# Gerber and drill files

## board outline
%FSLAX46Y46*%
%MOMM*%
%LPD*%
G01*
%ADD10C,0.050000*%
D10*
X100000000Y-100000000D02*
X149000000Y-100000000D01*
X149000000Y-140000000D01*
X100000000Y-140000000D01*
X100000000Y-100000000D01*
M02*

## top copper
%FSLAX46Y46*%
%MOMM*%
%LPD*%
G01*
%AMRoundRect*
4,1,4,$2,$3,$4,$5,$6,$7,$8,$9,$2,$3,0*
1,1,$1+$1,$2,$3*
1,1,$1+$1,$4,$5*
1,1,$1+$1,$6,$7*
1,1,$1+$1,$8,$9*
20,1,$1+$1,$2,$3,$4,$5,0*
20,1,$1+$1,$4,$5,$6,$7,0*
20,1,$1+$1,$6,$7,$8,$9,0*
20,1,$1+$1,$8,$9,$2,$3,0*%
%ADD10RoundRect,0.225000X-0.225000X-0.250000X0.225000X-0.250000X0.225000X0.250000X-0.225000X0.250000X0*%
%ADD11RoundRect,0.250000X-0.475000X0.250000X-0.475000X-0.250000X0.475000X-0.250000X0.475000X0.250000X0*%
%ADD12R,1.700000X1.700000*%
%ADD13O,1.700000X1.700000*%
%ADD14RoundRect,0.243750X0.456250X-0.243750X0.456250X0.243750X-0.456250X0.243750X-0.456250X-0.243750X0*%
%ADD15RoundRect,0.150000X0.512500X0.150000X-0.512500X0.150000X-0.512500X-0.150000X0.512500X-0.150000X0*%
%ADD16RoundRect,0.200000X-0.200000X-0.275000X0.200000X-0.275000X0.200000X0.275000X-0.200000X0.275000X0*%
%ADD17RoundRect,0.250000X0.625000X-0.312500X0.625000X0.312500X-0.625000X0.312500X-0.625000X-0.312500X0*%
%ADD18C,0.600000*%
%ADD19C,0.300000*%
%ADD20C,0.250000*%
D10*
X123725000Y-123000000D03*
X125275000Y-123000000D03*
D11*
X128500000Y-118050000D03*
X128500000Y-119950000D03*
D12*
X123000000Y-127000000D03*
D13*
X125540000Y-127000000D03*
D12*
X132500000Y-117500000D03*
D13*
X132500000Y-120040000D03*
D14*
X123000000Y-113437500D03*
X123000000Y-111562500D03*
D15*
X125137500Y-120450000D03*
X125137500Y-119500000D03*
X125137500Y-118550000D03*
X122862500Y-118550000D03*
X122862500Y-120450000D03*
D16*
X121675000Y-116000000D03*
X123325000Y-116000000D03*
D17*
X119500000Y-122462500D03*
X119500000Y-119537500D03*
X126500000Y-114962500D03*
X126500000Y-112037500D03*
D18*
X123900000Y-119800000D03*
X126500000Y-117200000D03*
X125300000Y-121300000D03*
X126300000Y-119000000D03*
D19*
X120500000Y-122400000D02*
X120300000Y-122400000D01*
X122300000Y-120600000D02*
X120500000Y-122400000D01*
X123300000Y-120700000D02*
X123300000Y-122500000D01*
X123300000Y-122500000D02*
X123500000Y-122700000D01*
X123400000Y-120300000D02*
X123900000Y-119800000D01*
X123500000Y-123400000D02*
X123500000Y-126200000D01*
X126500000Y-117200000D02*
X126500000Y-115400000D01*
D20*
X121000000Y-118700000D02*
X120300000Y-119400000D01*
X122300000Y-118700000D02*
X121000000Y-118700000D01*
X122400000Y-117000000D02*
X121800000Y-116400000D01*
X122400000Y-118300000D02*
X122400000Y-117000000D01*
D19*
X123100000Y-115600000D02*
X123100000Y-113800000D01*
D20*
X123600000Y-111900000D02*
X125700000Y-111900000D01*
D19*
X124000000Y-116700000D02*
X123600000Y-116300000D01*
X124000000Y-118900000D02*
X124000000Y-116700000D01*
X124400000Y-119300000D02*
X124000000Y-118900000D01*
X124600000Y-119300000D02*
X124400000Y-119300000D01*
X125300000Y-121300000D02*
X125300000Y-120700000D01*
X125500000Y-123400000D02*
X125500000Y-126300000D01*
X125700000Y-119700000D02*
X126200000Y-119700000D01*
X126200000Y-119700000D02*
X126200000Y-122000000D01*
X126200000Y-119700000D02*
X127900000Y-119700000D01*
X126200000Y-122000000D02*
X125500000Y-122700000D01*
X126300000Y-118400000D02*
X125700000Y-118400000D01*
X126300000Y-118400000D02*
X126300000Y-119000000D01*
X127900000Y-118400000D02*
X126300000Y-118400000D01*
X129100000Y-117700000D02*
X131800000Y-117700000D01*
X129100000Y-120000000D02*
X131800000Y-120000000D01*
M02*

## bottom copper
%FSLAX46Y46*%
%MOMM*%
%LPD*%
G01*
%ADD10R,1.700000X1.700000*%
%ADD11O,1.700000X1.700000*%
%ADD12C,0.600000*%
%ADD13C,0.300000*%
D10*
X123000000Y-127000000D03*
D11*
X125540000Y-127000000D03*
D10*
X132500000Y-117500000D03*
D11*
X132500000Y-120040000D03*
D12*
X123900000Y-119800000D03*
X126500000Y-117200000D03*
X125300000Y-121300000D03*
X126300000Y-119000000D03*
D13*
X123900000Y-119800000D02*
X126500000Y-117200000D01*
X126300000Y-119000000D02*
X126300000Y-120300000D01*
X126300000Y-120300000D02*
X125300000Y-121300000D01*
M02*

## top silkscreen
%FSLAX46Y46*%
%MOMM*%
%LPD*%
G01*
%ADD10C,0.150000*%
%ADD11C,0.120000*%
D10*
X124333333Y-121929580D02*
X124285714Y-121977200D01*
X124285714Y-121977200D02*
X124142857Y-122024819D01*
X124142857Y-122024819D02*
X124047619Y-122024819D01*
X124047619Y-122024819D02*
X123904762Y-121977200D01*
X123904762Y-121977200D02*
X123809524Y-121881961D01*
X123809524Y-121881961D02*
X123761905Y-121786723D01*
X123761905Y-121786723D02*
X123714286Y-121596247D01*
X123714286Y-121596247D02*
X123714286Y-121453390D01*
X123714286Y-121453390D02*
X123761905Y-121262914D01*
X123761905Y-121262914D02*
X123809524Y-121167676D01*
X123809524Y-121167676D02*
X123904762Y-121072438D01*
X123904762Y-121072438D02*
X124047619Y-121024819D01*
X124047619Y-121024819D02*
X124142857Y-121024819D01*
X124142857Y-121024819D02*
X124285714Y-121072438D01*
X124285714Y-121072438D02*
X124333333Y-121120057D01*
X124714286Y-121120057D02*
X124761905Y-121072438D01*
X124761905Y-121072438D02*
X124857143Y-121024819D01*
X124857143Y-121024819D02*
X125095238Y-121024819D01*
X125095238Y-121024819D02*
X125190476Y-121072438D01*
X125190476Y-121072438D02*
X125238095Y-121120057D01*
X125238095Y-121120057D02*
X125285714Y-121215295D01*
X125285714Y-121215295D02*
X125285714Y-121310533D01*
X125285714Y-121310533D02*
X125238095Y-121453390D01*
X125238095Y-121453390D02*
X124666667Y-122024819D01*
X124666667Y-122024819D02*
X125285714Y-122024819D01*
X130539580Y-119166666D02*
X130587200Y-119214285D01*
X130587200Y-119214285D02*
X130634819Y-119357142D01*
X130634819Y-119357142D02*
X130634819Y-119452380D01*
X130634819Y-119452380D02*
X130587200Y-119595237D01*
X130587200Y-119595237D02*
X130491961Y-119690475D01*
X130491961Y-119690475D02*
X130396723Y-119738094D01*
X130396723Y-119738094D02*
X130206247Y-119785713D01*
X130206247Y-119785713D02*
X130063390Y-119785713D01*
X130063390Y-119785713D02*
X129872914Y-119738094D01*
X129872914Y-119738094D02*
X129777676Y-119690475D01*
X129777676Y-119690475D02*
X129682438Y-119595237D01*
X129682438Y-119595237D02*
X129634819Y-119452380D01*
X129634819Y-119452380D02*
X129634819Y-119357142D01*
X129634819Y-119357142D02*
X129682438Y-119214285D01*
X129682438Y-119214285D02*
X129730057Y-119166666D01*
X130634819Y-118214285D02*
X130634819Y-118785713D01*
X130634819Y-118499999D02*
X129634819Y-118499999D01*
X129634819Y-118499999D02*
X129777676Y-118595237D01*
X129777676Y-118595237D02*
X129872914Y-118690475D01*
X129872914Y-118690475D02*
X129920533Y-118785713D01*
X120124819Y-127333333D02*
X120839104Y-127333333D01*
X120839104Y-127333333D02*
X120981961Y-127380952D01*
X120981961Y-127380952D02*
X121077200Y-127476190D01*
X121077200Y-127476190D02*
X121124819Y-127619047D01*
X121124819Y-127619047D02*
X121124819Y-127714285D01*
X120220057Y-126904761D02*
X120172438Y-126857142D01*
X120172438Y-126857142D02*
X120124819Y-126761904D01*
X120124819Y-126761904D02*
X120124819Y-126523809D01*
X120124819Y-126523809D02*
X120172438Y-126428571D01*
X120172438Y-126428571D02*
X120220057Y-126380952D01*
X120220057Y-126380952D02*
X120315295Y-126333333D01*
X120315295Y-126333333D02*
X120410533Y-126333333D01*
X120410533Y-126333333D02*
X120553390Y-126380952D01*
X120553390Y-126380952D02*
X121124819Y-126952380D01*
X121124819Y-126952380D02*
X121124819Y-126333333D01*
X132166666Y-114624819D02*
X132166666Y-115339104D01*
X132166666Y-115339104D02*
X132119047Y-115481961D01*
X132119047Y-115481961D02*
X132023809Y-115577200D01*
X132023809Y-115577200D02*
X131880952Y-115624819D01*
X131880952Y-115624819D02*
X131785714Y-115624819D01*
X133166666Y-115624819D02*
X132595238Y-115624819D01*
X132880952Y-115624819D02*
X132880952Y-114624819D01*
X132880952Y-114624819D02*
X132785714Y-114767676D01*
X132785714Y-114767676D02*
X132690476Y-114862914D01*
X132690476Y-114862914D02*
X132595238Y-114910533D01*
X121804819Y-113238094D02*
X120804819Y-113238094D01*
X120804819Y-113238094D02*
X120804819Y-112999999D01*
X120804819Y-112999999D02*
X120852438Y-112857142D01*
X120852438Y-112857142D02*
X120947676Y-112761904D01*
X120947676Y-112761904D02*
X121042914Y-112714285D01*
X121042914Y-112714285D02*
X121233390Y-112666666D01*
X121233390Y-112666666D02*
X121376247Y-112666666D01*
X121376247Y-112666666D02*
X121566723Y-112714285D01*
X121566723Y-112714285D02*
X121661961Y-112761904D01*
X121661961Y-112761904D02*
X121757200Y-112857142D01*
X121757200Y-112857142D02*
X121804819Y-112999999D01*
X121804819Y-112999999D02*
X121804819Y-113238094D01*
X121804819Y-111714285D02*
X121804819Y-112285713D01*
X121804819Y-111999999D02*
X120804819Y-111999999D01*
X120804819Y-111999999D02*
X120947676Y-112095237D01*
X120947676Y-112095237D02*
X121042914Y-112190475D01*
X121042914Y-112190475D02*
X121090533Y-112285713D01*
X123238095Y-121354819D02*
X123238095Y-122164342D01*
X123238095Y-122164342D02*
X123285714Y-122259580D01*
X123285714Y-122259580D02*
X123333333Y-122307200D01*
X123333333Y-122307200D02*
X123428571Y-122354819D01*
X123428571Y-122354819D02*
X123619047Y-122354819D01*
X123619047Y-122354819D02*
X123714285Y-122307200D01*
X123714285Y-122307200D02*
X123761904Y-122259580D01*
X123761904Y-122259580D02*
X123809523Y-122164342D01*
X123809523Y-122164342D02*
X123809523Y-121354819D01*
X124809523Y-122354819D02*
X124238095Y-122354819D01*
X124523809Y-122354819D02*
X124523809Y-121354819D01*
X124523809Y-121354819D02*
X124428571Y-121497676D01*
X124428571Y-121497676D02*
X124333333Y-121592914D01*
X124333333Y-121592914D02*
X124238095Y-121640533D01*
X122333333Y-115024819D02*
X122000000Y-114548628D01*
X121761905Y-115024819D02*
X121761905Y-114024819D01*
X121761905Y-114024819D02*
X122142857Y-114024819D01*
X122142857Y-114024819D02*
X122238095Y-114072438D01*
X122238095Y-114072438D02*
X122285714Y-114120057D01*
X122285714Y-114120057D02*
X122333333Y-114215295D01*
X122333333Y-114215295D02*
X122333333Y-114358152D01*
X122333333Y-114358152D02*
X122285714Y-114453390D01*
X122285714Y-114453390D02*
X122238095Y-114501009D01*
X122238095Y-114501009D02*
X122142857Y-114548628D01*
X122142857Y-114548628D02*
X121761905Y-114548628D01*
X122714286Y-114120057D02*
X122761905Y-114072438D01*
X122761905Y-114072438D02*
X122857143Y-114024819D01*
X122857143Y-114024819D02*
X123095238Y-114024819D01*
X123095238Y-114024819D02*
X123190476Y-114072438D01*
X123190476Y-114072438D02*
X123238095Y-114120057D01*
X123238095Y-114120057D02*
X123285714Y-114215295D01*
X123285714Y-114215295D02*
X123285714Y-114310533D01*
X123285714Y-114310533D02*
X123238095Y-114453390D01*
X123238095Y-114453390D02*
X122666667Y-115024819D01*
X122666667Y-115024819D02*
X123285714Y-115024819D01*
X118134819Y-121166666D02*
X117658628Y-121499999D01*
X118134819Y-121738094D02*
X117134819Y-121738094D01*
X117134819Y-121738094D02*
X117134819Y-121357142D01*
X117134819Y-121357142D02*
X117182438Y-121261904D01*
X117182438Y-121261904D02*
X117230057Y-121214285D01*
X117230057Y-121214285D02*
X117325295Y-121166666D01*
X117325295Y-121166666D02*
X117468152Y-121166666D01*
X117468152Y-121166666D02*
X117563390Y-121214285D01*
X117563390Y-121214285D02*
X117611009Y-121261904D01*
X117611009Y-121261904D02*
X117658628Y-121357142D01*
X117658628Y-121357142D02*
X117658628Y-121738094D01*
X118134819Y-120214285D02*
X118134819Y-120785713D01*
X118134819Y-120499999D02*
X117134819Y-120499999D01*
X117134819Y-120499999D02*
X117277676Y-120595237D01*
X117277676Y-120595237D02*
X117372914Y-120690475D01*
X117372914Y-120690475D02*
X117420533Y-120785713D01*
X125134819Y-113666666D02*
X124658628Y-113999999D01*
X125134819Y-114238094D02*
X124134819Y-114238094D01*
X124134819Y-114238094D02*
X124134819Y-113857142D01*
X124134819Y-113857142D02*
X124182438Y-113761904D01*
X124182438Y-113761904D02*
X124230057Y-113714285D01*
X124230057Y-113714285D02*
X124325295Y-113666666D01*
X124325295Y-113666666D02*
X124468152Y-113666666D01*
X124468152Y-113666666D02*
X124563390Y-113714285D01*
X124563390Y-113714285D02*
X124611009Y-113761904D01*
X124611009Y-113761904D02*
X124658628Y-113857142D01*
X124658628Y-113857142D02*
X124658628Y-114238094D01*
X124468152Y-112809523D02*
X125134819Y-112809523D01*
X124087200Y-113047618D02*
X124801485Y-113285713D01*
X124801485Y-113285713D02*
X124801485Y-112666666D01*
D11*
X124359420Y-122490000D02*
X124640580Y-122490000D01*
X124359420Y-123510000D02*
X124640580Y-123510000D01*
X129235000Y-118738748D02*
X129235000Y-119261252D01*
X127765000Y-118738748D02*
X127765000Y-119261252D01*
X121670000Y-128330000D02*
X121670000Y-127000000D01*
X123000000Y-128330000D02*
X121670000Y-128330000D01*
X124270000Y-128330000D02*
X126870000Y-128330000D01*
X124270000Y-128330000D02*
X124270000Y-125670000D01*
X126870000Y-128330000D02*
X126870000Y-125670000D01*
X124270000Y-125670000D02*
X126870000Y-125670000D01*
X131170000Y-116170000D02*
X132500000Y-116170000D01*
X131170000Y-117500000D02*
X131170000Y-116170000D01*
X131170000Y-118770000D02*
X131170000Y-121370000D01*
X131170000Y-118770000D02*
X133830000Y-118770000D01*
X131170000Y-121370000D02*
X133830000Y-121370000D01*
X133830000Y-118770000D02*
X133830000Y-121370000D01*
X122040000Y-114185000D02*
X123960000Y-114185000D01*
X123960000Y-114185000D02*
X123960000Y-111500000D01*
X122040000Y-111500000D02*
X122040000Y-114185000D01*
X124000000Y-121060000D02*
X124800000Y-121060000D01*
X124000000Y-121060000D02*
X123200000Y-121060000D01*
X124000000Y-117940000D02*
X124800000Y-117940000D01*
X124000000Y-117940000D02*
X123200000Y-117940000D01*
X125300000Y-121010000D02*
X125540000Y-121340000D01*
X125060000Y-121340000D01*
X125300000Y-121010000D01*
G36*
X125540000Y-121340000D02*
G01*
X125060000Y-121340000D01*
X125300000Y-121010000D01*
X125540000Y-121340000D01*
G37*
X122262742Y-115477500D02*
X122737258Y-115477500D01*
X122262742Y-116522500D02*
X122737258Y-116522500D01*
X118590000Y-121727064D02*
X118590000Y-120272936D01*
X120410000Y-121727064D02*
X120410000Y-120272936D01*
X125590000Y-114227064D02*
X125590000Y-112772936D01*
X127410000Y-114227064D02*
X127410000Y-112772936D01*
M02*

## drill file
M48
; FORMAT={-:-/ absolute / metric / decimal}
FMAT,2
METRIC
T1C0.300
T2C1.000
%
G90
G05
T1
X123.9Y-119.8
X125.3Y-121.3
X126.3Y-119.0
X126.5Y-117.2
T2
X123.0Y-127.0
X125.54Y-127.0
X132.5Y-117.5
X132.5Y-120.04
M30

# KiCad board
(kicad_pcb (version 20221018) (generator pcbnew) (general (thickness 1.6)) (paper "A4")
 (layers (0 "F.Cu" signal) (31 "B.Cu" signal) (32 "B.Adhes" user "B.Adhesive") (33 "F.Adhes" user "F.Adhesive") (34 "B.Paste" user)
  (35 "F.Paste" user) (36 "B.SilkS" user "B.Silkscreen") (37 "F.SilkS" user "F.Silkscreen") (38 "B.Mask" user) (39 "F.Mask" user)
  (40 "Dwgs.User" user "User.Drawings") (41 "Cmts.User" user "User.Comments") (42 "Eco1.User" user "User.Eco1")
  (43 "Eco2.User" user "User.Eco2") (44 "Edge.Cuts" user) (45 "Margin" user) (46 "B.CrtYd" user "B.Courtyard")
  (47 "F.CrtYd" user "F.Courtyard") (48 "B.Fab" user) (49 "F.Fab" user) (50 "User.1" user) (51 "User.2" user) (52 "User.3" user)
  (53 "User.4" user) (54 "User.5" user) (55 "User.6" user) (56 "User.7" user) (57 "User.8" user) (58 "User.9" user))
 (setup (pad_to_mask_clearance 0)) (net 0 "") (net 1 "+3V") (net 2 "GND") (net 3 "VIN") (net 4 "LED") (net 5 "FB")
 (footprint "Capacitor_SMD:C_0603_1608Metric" (layer "F.Cu") (at 124.5 123)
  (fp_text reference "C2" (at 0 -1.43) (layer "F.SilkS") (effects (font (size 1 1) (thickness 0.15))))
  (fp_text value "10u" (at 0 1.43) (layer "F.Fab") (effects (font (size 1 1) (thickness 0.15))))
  (fp_line (start -0.14058 -0.51) (end 0.14058 -0.51) (stroke (width 0.12) (type solid)) (layer "F.SilkS"))
  (fp_line (start -0.14058 0.51) (end 0.14058 0.51) (stroke (width 0.12) (type solid)) (layer "F.SilkS"))
  (pad "1" smd roundrect (at -0.775 0) (size 0.9 0.95) (layers "F.Cu" "F.Paste" "F.Mask") (roundrect_rratio 0.25) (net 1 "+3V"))
  (pad "2" smd roundrect (at 0.775 0) (size 0.9 0.95) (layers "F.Cu" "F.Paste" "F.Mask") (roundrect_rratio 0.25) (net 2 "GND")))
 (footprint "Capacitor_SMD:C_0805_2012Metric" (layer "F.Cu") (at 128.5 119 -90)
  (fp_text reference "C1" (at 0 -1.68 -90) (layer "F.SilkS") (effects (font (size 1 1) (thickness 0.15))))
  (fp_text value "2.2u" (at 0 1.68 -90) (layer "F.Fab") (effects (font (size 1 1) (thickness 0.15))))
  (fp_line (start -0.261252 -0.735) (end 0.261252 -0.735) (stroke (width 0.12) (type solid)) (layer "F.SilkS"))
  (fp_line (start -0.261252 0.735) (end 0.261252 0.735) (stroke (width 0.12) (type solid)) (layer "F.SilkS"))
  (pad "1" smd roundrect (at -0.95 0 270) (size 1 1.45) (layers "F.Cu" "F.Paste" "F.Mask") (roundrect_rratio 0.25) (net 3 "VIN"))
  (pad "2" smd roundrect (at 0.95 0 270) (size 1 1.45) (layers "F.Cu" "F.Paste" "F.Mask") (roundrect_rratio 0.25) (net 2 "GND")))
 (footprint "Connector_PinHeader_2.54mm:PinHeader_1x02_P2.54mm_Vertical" (layer "F.Cu") (at 123 127 90)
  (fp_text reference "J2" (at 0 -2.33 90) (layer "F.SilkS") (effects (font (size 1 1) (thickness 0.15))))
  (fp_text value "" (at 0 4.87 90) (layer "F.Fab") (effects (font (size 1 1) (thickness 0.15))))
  (fp_line (start -1.33 -1.33) (end 0 -1.33) (stroke (width 0.12) (type solid)) (layer "F.SilkS"))
  (fp_line (start -1.33 0) (end -1.33 -1.33) (stroke (width 0.12) (type solid)) (layer "F.SilkS"))
  (fp_line (start -1.33 1.27) (end -1.33 3.87) (stroke (width 0.12) (type solid)) (layer "F.SilkS"))
  (fp_line (start -1.33 1.27) (end 1.33 1.27) (stroke (width 0.12) (type solid)) (layer "F.SilkS"))
  (fp_line (start -1.33 3.87) (end 1.33 3.87) (stroke (width 0.12) (type solid)) (layer "F.SilkS"))
  (fp_line (start 1.33 1.27) (end 1.33 3.87) (stroke (width 0.12) (type solid)) (layer "F.SilkS"))
  (pad "1" thru_hole rect (at 0 0 90) (size 1.7 1.7) (drill 1) (layers "*.Cu" "*.Mask") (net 1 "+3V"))
  (pad "2" thru_hole oval (at 0 2.54 90) (size 1.7 1.7) (drill 1) (layers "*.Cu" "*.Mask") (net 2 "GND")))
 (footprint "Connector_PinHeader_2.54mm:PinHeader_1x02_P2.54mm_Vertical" (layer "F.Cu") (at 132.5 117.5)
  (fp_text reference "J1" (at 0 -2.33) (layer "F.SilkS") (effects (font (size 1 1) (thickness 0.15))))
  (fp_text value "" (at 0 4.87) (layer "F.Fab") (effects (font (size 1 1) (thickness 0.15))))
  (fp_line (start -1.33 -1.33) (end 0 -1.33) (stroke (width 0.12) (type solid)) (layer "F.SilkS"))
  (fp_line (start -1.33 0) (end -1.33 -1.33) (stroke (width 0.12) (type solid)) (layer "F.SilkS"))
  (fp_line (start -1.33 1.27) (end -1.33 3.87) (stroke (width 0.12) (type solid)) (layer "F.SilkS"))
  (fp_line (start -1.33 1.27) (end 1.33 1.27) (stroke (width 0.12) (type solid)) (layer "F.SilkS"))
  (fp_line (start -1.33 3.87) (end 1.33 3.87) (stroke (width 0.12) (type solid)) (layer "F.SilkS"))
  (fp_line (start 1.33 1.27) (end 1.33 3.87) (stroke (width 0.12) (type solid)) (layer "F.SilkS"))
  (pad "1" thru_hole rect (at 0 0) (size 1.7 1.7) (drill 1) (layers "*.Cu" "*.Mask") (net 3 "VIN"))
  (pad "2" thru_hole oval (at 0 2.54) (size 1.7 1.7) (drill 1) (layers "*.Cu" "*.Mask") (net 2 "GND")))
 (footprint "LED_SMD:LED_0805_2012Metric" (layer "F.Cu") (at 123 112.5 90)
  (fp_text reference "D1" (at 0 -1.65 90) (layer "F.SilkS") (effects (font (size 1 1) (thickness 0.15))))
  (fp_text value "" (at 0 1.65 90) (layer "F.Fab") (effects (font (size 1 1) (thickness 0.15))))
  (fp_line (start -1.685 -0.96) (end -1.685 0.96) (stroke (width 0.12) (type solid)) (layer "F.SilkS"))
  (fp_line (start -1.685 0.96) (end 1 0.96) (stroke (width 0.12) (type solid)) (layer "F.SilkS"))
  (fp_line (start 1 -0.96) (end -1.685 -0.96) (stroke (width 0.12) (type solid)) (layer "F.SilkS"))
  (pad "1" smd roundrect (at -0.9375 0 90) (size 0.975 1.4) (layers "F.Cu" "F.Paste" "F.Mask") (roundrect_rratio 0.25) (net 2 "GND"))
  (pad "2" smd roundrect (at 0.9375 0 90) (size 0.975 1.4) (layers "F.Cu" "F.Paste" "F.Mask") (roundrect_rratio 0.25) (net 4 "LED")))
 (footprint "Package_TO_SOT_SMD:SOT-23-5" (layer "F.Cu") (at 124 119.5 180)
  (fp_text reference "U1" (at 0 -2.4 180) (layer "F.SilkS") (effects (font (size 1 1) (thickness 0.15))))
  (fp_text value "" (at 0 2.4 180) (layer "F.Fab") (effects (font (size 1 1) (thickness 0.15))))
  (fp_line (start 0 -1.56) (end -0.8 -1.56) (stroke (width 0.12) (type solid)) (layer "F.SilkS"))
  (fp_line (start 0 -1.56) (end 0.8 -1.56) (stroke (width 0.12) (type solid)) (layer "F.SilkS"))
  (fp_line (start 0 1.56) (end -0.8 1.56) (stroke (width 0.12) (type solid)) (layer "F.SilkS"))
  (fp_line (start 0 1.56) (end 0.8 1.56) (stroke (width 0.12) (type solid)) (layer "F.SilkS"))
  (fp_poly
   (pts (xy -1.3 -1.51) (xy -1.54 -1.84) (xy -1.06 -1.84) (xy -1.3 -1.51)) (stroke (width 0.12) (type solid)) (fill solid) (layer "F.SilkS"))
  (pad "1" smd roundrect (at -1.1375 -0.95 180) (size 1.325 0.6) (layers "F.Cu" "F.Paste" "F.Mask") (roundrect_rratio 0.25) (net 3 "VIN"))
  (pad "2" smd roundrect (at -1.1375 0 180) (size 1.325 0.6) (layers "F.Cu" "F.Paste" "F.Mask") (roundrect_rratio 0.25) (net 2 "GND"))
  (pad "3" smd roundrect (at -1.1375 0.95 180) (size 1.325 0.6) (layers "F.Cu" "F.Paste" "F.Mask") (roundrect_rratio 0.25) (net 3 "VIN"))
  (pad "4" smd roundrect (at 1.1375 0.95 180) (size 1.325 0.6) (layers "F.Cu" "F.Paste" "F.Mask") (roundrect_rratio 0.25) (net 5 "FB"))
  (pad "5" smd roundrect (at 1.1375 -0.95 180) (size 1.325 0.6) (layers "F.Cu" "F.Paste" "F.Mask") (roundrect_rratio 0.25) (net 1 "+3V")))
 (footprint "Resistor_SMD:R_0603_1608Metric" (layer "F.Cu") (at 122.5 116)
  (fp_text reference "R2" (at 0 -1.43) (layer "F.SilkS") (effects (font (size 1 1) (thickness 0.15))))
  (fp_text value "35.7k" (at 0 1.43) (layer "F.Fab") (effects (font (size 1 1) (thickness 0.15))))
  (fp_line (start -0.237258 -0.5225) (end 0.237258 -0.5225) (stroke (width 0.12) (type solid)) (layer "F.SilkS"))
  (fp_line (start -0.237258 0.5225) (end 0.237258 0.5225) (stroke (width 0.12) (type solid)) (layer "F.SilkS"))
  (pad "1" smd roundrect (at -0.825 0) (size 0.8 0.95) (layers "F.Cu" "F.Paste" "F.Mask") (roundrect_rratio 0.25) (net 5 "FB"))
  (pad "2" smd roundrect (at 0.825 0) (size 0.8 0.95) (layers "F.Cu" "F.Paste" "F.Mask") (roundrect_rratio 0.25) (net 2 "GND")))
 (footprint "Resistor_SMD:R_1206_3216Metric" (layer "F.Cu") (at 119.5 121 90)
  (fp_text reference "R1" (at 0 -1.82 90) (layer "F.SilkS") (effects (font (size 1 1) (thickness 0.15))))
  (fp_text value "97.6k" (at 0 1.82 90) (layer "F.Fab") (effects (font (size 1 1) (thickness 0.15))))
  (fp_line (start -0.727064 -0.91) (end 0.727064 -0.91) (stroke (width 0.12) (type solid)) (layer "F.SilkS"))
  (fp_line (start -0.727064 0.91) (end 0.727064 0.91) (stroke (width 0.12) (type solid)) (layer "F.SilkS"))
  (pad "1" smd roundrect (at -1.4625 0 90) (size 1.125 1.75) (layers "F.Cu" "F.Paste" "F.Mask") (roundrect_rratio 0.222222) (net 1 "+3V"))
  (pad "2" smd roundrect (at 1.4625 0 90) (size 1.125 1.75) (layers "F.Cu" "F.Paste" "F.Mask") (roundrect_rratio 0.222222) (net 5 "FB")))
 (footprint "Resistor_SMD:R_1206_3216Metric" (layer "F.Cu") (at 126.5 113.5 90)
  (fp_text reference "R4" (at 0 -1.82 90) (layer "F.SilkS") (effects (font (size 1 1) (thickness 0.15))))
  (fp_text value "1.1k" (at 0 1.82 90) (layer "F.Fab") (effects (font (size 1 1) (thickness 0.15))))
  (fp_line (start -0.727064 -0.91) (end 0.727064 -0.91) (stroke (width 0.12) (type solid)) (layer "F.SilkS"))
  (fp_line (start -0.727064 0.91) (end 0.727064 0.91) (stroke (width 0.12) (type solid)) (layer "F.SilkS"))
  (pad "1" smd roundrect (at -1.4625 0 90) (size 1.125 1.75) (layers "F.Cu" "F.Paste" "F.Mask") (roundrect_rratio 0.222222) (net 1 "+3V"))
  (pad "2" smd roundrect (at 1.4625 0 90) (size 1.125 1.75) (layers "F.Cu" "F.Paste" "F.Mask") (roundrect_rratio 0.222222) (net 4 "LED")))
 (gr_rect (start 100 100) (end 149 140) (stroke (width 0.05) (type default)) (fill none) (layer "Edge.Cuts"))
 (segment (start 120.5 122.4) (end 120.3 122.4) (width 0.3) (layer "F.Cu") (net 1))
 (segment (start 122.3 120.6) (end 120.5 122.4) (width 0.3) (layer "F.Cu") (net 1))
 (segment (start 123.3 120.7) (end 123.3 122.5) (width 0.3) (layer "F.Cu") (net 1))
 (segment (start 123.3 122.5) (end 123.5 122.7) (width 0.3) (layer "F.Cu") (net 1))
 (segment (start 123.4 120.3) (end 123.9 119.8) (width 0.3) (layer "F.Cu") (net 1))
 (segment (start 123.5 123.4) (end 123.5 126.2) (width 0.3) (layer "F.Cu") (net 1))
 (segment (start 126.5 117.2) (end 126.5 115.4) (width 0.3) (layer "F.Cu") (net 1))
 (via (at 123.9 119.8) (size 0.6) (drill 0.3) (layers "F.Cu" "B.Cu") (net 1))
 (via (at 126.5 117.2) (size 0.6) (drill 0.3) (layers "F.Cu" "B.Cu") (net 1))
 (segment (start 121 118.7) (end 120.3 119.4) (width 0.25) (layer "F.Cu") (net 5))
 (segment (start 122.3 118.7) (end 121 118.7) (width 0.25) (layer "F.Cu") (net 5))
 (segment (start 122.4 117) (end 121.8 116.4) (width 0.25) (layer "F.Cu") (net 5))
 (segment (start 122.4 118.3) (end 122.4 117) (width 0.25) (layer "F.Cu") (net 5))
 (segment (start 123.1 115.6) (end 123.1 113.8) (width 0.3) (layer "F.Cu") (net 2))
 (segment (start 123.6 111.9) (end 125.7 111.9) (width 0.25) (layer "F.Cu") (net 4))
 (segment (start 123.9 119.8) (end 126.5 117.2) (width 0.3) (layer "B.Cu") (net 1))
 (segment (start 124 116.7) (end 123.6 116.3) (width 0.3) (layer "F.Cu") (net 2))
 (segment (start 124 118.9) (end 124 116.7) (width 0.3) (layer "F.Cu") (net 2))
 (segment (start 124.4 119.3) (end 124 118.9) (width 0.3) (layer "F.Cu") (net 2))
 (segment (start 124.6 119.3) (end 124.4 119.3) (width 0.3) (layer "F.Cu") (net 2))
 (segment (start 125.3 121.3) (end 125.3 120.7) (width 0.3) (layer "F.Cu") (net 3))
 (segment (start 125.5 123.4) (end 125.5 126.3) (width 0.3) (layer "F.Cu") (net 2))
 (segment (start 125.7 119.7) (end 126.2 119.7) (width 0.3) (layer "F.Cu") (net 2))
 (segment (start 126.2 119.7) (end 126.2 122) (width 0.3) (layer "F.Cu") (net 2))
 (segment (start 126.2 119.7) (end 127.9 119.7) (width 0.3) (layer "F.Cu") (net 2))
 (segment (start 126.2 122) (end 125.5 122.7) (width 0.3) (layer "F.Cu") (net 2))
 (segment (start 126.3 118.4) (end 125.7 118.4) (width 0.3) (layer "F.Cu") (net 3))
 (segment (start 126.3 118.4) (end 126.3 119) (width 0.3) (layer "F.Cu") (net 3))
 (segment (start 127.9 118.4) (end 126.3 118.4) (width 0.3) (layer "F.Cu") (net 3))
 (segment (start 129.1 117.7) (end 131.8 117.7) (width 0.3) (layer "F.Cu") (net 3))
 (segment (start 129.1 120) (end 131.8 120) (width 0.3) (layer "F.Cu") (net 2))
 (via (at 125.3 121.3) (size 0.6) (drill 0.3) (layers "F.Cu" "B.Cu") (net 3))
 (via (at 126.3 119) (size 0.6) (drill 0.3) (layers "F.Cu" "B.Cu") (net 3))
 (segment (start 126.3 119) (end 126.3 120.3) (width 0.3) (layer "B.Cu") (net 3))
 (segment (start 126.3 120.3) (end 125.3 121.3) (width 0.3) (layer "B.Cu") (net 3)))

